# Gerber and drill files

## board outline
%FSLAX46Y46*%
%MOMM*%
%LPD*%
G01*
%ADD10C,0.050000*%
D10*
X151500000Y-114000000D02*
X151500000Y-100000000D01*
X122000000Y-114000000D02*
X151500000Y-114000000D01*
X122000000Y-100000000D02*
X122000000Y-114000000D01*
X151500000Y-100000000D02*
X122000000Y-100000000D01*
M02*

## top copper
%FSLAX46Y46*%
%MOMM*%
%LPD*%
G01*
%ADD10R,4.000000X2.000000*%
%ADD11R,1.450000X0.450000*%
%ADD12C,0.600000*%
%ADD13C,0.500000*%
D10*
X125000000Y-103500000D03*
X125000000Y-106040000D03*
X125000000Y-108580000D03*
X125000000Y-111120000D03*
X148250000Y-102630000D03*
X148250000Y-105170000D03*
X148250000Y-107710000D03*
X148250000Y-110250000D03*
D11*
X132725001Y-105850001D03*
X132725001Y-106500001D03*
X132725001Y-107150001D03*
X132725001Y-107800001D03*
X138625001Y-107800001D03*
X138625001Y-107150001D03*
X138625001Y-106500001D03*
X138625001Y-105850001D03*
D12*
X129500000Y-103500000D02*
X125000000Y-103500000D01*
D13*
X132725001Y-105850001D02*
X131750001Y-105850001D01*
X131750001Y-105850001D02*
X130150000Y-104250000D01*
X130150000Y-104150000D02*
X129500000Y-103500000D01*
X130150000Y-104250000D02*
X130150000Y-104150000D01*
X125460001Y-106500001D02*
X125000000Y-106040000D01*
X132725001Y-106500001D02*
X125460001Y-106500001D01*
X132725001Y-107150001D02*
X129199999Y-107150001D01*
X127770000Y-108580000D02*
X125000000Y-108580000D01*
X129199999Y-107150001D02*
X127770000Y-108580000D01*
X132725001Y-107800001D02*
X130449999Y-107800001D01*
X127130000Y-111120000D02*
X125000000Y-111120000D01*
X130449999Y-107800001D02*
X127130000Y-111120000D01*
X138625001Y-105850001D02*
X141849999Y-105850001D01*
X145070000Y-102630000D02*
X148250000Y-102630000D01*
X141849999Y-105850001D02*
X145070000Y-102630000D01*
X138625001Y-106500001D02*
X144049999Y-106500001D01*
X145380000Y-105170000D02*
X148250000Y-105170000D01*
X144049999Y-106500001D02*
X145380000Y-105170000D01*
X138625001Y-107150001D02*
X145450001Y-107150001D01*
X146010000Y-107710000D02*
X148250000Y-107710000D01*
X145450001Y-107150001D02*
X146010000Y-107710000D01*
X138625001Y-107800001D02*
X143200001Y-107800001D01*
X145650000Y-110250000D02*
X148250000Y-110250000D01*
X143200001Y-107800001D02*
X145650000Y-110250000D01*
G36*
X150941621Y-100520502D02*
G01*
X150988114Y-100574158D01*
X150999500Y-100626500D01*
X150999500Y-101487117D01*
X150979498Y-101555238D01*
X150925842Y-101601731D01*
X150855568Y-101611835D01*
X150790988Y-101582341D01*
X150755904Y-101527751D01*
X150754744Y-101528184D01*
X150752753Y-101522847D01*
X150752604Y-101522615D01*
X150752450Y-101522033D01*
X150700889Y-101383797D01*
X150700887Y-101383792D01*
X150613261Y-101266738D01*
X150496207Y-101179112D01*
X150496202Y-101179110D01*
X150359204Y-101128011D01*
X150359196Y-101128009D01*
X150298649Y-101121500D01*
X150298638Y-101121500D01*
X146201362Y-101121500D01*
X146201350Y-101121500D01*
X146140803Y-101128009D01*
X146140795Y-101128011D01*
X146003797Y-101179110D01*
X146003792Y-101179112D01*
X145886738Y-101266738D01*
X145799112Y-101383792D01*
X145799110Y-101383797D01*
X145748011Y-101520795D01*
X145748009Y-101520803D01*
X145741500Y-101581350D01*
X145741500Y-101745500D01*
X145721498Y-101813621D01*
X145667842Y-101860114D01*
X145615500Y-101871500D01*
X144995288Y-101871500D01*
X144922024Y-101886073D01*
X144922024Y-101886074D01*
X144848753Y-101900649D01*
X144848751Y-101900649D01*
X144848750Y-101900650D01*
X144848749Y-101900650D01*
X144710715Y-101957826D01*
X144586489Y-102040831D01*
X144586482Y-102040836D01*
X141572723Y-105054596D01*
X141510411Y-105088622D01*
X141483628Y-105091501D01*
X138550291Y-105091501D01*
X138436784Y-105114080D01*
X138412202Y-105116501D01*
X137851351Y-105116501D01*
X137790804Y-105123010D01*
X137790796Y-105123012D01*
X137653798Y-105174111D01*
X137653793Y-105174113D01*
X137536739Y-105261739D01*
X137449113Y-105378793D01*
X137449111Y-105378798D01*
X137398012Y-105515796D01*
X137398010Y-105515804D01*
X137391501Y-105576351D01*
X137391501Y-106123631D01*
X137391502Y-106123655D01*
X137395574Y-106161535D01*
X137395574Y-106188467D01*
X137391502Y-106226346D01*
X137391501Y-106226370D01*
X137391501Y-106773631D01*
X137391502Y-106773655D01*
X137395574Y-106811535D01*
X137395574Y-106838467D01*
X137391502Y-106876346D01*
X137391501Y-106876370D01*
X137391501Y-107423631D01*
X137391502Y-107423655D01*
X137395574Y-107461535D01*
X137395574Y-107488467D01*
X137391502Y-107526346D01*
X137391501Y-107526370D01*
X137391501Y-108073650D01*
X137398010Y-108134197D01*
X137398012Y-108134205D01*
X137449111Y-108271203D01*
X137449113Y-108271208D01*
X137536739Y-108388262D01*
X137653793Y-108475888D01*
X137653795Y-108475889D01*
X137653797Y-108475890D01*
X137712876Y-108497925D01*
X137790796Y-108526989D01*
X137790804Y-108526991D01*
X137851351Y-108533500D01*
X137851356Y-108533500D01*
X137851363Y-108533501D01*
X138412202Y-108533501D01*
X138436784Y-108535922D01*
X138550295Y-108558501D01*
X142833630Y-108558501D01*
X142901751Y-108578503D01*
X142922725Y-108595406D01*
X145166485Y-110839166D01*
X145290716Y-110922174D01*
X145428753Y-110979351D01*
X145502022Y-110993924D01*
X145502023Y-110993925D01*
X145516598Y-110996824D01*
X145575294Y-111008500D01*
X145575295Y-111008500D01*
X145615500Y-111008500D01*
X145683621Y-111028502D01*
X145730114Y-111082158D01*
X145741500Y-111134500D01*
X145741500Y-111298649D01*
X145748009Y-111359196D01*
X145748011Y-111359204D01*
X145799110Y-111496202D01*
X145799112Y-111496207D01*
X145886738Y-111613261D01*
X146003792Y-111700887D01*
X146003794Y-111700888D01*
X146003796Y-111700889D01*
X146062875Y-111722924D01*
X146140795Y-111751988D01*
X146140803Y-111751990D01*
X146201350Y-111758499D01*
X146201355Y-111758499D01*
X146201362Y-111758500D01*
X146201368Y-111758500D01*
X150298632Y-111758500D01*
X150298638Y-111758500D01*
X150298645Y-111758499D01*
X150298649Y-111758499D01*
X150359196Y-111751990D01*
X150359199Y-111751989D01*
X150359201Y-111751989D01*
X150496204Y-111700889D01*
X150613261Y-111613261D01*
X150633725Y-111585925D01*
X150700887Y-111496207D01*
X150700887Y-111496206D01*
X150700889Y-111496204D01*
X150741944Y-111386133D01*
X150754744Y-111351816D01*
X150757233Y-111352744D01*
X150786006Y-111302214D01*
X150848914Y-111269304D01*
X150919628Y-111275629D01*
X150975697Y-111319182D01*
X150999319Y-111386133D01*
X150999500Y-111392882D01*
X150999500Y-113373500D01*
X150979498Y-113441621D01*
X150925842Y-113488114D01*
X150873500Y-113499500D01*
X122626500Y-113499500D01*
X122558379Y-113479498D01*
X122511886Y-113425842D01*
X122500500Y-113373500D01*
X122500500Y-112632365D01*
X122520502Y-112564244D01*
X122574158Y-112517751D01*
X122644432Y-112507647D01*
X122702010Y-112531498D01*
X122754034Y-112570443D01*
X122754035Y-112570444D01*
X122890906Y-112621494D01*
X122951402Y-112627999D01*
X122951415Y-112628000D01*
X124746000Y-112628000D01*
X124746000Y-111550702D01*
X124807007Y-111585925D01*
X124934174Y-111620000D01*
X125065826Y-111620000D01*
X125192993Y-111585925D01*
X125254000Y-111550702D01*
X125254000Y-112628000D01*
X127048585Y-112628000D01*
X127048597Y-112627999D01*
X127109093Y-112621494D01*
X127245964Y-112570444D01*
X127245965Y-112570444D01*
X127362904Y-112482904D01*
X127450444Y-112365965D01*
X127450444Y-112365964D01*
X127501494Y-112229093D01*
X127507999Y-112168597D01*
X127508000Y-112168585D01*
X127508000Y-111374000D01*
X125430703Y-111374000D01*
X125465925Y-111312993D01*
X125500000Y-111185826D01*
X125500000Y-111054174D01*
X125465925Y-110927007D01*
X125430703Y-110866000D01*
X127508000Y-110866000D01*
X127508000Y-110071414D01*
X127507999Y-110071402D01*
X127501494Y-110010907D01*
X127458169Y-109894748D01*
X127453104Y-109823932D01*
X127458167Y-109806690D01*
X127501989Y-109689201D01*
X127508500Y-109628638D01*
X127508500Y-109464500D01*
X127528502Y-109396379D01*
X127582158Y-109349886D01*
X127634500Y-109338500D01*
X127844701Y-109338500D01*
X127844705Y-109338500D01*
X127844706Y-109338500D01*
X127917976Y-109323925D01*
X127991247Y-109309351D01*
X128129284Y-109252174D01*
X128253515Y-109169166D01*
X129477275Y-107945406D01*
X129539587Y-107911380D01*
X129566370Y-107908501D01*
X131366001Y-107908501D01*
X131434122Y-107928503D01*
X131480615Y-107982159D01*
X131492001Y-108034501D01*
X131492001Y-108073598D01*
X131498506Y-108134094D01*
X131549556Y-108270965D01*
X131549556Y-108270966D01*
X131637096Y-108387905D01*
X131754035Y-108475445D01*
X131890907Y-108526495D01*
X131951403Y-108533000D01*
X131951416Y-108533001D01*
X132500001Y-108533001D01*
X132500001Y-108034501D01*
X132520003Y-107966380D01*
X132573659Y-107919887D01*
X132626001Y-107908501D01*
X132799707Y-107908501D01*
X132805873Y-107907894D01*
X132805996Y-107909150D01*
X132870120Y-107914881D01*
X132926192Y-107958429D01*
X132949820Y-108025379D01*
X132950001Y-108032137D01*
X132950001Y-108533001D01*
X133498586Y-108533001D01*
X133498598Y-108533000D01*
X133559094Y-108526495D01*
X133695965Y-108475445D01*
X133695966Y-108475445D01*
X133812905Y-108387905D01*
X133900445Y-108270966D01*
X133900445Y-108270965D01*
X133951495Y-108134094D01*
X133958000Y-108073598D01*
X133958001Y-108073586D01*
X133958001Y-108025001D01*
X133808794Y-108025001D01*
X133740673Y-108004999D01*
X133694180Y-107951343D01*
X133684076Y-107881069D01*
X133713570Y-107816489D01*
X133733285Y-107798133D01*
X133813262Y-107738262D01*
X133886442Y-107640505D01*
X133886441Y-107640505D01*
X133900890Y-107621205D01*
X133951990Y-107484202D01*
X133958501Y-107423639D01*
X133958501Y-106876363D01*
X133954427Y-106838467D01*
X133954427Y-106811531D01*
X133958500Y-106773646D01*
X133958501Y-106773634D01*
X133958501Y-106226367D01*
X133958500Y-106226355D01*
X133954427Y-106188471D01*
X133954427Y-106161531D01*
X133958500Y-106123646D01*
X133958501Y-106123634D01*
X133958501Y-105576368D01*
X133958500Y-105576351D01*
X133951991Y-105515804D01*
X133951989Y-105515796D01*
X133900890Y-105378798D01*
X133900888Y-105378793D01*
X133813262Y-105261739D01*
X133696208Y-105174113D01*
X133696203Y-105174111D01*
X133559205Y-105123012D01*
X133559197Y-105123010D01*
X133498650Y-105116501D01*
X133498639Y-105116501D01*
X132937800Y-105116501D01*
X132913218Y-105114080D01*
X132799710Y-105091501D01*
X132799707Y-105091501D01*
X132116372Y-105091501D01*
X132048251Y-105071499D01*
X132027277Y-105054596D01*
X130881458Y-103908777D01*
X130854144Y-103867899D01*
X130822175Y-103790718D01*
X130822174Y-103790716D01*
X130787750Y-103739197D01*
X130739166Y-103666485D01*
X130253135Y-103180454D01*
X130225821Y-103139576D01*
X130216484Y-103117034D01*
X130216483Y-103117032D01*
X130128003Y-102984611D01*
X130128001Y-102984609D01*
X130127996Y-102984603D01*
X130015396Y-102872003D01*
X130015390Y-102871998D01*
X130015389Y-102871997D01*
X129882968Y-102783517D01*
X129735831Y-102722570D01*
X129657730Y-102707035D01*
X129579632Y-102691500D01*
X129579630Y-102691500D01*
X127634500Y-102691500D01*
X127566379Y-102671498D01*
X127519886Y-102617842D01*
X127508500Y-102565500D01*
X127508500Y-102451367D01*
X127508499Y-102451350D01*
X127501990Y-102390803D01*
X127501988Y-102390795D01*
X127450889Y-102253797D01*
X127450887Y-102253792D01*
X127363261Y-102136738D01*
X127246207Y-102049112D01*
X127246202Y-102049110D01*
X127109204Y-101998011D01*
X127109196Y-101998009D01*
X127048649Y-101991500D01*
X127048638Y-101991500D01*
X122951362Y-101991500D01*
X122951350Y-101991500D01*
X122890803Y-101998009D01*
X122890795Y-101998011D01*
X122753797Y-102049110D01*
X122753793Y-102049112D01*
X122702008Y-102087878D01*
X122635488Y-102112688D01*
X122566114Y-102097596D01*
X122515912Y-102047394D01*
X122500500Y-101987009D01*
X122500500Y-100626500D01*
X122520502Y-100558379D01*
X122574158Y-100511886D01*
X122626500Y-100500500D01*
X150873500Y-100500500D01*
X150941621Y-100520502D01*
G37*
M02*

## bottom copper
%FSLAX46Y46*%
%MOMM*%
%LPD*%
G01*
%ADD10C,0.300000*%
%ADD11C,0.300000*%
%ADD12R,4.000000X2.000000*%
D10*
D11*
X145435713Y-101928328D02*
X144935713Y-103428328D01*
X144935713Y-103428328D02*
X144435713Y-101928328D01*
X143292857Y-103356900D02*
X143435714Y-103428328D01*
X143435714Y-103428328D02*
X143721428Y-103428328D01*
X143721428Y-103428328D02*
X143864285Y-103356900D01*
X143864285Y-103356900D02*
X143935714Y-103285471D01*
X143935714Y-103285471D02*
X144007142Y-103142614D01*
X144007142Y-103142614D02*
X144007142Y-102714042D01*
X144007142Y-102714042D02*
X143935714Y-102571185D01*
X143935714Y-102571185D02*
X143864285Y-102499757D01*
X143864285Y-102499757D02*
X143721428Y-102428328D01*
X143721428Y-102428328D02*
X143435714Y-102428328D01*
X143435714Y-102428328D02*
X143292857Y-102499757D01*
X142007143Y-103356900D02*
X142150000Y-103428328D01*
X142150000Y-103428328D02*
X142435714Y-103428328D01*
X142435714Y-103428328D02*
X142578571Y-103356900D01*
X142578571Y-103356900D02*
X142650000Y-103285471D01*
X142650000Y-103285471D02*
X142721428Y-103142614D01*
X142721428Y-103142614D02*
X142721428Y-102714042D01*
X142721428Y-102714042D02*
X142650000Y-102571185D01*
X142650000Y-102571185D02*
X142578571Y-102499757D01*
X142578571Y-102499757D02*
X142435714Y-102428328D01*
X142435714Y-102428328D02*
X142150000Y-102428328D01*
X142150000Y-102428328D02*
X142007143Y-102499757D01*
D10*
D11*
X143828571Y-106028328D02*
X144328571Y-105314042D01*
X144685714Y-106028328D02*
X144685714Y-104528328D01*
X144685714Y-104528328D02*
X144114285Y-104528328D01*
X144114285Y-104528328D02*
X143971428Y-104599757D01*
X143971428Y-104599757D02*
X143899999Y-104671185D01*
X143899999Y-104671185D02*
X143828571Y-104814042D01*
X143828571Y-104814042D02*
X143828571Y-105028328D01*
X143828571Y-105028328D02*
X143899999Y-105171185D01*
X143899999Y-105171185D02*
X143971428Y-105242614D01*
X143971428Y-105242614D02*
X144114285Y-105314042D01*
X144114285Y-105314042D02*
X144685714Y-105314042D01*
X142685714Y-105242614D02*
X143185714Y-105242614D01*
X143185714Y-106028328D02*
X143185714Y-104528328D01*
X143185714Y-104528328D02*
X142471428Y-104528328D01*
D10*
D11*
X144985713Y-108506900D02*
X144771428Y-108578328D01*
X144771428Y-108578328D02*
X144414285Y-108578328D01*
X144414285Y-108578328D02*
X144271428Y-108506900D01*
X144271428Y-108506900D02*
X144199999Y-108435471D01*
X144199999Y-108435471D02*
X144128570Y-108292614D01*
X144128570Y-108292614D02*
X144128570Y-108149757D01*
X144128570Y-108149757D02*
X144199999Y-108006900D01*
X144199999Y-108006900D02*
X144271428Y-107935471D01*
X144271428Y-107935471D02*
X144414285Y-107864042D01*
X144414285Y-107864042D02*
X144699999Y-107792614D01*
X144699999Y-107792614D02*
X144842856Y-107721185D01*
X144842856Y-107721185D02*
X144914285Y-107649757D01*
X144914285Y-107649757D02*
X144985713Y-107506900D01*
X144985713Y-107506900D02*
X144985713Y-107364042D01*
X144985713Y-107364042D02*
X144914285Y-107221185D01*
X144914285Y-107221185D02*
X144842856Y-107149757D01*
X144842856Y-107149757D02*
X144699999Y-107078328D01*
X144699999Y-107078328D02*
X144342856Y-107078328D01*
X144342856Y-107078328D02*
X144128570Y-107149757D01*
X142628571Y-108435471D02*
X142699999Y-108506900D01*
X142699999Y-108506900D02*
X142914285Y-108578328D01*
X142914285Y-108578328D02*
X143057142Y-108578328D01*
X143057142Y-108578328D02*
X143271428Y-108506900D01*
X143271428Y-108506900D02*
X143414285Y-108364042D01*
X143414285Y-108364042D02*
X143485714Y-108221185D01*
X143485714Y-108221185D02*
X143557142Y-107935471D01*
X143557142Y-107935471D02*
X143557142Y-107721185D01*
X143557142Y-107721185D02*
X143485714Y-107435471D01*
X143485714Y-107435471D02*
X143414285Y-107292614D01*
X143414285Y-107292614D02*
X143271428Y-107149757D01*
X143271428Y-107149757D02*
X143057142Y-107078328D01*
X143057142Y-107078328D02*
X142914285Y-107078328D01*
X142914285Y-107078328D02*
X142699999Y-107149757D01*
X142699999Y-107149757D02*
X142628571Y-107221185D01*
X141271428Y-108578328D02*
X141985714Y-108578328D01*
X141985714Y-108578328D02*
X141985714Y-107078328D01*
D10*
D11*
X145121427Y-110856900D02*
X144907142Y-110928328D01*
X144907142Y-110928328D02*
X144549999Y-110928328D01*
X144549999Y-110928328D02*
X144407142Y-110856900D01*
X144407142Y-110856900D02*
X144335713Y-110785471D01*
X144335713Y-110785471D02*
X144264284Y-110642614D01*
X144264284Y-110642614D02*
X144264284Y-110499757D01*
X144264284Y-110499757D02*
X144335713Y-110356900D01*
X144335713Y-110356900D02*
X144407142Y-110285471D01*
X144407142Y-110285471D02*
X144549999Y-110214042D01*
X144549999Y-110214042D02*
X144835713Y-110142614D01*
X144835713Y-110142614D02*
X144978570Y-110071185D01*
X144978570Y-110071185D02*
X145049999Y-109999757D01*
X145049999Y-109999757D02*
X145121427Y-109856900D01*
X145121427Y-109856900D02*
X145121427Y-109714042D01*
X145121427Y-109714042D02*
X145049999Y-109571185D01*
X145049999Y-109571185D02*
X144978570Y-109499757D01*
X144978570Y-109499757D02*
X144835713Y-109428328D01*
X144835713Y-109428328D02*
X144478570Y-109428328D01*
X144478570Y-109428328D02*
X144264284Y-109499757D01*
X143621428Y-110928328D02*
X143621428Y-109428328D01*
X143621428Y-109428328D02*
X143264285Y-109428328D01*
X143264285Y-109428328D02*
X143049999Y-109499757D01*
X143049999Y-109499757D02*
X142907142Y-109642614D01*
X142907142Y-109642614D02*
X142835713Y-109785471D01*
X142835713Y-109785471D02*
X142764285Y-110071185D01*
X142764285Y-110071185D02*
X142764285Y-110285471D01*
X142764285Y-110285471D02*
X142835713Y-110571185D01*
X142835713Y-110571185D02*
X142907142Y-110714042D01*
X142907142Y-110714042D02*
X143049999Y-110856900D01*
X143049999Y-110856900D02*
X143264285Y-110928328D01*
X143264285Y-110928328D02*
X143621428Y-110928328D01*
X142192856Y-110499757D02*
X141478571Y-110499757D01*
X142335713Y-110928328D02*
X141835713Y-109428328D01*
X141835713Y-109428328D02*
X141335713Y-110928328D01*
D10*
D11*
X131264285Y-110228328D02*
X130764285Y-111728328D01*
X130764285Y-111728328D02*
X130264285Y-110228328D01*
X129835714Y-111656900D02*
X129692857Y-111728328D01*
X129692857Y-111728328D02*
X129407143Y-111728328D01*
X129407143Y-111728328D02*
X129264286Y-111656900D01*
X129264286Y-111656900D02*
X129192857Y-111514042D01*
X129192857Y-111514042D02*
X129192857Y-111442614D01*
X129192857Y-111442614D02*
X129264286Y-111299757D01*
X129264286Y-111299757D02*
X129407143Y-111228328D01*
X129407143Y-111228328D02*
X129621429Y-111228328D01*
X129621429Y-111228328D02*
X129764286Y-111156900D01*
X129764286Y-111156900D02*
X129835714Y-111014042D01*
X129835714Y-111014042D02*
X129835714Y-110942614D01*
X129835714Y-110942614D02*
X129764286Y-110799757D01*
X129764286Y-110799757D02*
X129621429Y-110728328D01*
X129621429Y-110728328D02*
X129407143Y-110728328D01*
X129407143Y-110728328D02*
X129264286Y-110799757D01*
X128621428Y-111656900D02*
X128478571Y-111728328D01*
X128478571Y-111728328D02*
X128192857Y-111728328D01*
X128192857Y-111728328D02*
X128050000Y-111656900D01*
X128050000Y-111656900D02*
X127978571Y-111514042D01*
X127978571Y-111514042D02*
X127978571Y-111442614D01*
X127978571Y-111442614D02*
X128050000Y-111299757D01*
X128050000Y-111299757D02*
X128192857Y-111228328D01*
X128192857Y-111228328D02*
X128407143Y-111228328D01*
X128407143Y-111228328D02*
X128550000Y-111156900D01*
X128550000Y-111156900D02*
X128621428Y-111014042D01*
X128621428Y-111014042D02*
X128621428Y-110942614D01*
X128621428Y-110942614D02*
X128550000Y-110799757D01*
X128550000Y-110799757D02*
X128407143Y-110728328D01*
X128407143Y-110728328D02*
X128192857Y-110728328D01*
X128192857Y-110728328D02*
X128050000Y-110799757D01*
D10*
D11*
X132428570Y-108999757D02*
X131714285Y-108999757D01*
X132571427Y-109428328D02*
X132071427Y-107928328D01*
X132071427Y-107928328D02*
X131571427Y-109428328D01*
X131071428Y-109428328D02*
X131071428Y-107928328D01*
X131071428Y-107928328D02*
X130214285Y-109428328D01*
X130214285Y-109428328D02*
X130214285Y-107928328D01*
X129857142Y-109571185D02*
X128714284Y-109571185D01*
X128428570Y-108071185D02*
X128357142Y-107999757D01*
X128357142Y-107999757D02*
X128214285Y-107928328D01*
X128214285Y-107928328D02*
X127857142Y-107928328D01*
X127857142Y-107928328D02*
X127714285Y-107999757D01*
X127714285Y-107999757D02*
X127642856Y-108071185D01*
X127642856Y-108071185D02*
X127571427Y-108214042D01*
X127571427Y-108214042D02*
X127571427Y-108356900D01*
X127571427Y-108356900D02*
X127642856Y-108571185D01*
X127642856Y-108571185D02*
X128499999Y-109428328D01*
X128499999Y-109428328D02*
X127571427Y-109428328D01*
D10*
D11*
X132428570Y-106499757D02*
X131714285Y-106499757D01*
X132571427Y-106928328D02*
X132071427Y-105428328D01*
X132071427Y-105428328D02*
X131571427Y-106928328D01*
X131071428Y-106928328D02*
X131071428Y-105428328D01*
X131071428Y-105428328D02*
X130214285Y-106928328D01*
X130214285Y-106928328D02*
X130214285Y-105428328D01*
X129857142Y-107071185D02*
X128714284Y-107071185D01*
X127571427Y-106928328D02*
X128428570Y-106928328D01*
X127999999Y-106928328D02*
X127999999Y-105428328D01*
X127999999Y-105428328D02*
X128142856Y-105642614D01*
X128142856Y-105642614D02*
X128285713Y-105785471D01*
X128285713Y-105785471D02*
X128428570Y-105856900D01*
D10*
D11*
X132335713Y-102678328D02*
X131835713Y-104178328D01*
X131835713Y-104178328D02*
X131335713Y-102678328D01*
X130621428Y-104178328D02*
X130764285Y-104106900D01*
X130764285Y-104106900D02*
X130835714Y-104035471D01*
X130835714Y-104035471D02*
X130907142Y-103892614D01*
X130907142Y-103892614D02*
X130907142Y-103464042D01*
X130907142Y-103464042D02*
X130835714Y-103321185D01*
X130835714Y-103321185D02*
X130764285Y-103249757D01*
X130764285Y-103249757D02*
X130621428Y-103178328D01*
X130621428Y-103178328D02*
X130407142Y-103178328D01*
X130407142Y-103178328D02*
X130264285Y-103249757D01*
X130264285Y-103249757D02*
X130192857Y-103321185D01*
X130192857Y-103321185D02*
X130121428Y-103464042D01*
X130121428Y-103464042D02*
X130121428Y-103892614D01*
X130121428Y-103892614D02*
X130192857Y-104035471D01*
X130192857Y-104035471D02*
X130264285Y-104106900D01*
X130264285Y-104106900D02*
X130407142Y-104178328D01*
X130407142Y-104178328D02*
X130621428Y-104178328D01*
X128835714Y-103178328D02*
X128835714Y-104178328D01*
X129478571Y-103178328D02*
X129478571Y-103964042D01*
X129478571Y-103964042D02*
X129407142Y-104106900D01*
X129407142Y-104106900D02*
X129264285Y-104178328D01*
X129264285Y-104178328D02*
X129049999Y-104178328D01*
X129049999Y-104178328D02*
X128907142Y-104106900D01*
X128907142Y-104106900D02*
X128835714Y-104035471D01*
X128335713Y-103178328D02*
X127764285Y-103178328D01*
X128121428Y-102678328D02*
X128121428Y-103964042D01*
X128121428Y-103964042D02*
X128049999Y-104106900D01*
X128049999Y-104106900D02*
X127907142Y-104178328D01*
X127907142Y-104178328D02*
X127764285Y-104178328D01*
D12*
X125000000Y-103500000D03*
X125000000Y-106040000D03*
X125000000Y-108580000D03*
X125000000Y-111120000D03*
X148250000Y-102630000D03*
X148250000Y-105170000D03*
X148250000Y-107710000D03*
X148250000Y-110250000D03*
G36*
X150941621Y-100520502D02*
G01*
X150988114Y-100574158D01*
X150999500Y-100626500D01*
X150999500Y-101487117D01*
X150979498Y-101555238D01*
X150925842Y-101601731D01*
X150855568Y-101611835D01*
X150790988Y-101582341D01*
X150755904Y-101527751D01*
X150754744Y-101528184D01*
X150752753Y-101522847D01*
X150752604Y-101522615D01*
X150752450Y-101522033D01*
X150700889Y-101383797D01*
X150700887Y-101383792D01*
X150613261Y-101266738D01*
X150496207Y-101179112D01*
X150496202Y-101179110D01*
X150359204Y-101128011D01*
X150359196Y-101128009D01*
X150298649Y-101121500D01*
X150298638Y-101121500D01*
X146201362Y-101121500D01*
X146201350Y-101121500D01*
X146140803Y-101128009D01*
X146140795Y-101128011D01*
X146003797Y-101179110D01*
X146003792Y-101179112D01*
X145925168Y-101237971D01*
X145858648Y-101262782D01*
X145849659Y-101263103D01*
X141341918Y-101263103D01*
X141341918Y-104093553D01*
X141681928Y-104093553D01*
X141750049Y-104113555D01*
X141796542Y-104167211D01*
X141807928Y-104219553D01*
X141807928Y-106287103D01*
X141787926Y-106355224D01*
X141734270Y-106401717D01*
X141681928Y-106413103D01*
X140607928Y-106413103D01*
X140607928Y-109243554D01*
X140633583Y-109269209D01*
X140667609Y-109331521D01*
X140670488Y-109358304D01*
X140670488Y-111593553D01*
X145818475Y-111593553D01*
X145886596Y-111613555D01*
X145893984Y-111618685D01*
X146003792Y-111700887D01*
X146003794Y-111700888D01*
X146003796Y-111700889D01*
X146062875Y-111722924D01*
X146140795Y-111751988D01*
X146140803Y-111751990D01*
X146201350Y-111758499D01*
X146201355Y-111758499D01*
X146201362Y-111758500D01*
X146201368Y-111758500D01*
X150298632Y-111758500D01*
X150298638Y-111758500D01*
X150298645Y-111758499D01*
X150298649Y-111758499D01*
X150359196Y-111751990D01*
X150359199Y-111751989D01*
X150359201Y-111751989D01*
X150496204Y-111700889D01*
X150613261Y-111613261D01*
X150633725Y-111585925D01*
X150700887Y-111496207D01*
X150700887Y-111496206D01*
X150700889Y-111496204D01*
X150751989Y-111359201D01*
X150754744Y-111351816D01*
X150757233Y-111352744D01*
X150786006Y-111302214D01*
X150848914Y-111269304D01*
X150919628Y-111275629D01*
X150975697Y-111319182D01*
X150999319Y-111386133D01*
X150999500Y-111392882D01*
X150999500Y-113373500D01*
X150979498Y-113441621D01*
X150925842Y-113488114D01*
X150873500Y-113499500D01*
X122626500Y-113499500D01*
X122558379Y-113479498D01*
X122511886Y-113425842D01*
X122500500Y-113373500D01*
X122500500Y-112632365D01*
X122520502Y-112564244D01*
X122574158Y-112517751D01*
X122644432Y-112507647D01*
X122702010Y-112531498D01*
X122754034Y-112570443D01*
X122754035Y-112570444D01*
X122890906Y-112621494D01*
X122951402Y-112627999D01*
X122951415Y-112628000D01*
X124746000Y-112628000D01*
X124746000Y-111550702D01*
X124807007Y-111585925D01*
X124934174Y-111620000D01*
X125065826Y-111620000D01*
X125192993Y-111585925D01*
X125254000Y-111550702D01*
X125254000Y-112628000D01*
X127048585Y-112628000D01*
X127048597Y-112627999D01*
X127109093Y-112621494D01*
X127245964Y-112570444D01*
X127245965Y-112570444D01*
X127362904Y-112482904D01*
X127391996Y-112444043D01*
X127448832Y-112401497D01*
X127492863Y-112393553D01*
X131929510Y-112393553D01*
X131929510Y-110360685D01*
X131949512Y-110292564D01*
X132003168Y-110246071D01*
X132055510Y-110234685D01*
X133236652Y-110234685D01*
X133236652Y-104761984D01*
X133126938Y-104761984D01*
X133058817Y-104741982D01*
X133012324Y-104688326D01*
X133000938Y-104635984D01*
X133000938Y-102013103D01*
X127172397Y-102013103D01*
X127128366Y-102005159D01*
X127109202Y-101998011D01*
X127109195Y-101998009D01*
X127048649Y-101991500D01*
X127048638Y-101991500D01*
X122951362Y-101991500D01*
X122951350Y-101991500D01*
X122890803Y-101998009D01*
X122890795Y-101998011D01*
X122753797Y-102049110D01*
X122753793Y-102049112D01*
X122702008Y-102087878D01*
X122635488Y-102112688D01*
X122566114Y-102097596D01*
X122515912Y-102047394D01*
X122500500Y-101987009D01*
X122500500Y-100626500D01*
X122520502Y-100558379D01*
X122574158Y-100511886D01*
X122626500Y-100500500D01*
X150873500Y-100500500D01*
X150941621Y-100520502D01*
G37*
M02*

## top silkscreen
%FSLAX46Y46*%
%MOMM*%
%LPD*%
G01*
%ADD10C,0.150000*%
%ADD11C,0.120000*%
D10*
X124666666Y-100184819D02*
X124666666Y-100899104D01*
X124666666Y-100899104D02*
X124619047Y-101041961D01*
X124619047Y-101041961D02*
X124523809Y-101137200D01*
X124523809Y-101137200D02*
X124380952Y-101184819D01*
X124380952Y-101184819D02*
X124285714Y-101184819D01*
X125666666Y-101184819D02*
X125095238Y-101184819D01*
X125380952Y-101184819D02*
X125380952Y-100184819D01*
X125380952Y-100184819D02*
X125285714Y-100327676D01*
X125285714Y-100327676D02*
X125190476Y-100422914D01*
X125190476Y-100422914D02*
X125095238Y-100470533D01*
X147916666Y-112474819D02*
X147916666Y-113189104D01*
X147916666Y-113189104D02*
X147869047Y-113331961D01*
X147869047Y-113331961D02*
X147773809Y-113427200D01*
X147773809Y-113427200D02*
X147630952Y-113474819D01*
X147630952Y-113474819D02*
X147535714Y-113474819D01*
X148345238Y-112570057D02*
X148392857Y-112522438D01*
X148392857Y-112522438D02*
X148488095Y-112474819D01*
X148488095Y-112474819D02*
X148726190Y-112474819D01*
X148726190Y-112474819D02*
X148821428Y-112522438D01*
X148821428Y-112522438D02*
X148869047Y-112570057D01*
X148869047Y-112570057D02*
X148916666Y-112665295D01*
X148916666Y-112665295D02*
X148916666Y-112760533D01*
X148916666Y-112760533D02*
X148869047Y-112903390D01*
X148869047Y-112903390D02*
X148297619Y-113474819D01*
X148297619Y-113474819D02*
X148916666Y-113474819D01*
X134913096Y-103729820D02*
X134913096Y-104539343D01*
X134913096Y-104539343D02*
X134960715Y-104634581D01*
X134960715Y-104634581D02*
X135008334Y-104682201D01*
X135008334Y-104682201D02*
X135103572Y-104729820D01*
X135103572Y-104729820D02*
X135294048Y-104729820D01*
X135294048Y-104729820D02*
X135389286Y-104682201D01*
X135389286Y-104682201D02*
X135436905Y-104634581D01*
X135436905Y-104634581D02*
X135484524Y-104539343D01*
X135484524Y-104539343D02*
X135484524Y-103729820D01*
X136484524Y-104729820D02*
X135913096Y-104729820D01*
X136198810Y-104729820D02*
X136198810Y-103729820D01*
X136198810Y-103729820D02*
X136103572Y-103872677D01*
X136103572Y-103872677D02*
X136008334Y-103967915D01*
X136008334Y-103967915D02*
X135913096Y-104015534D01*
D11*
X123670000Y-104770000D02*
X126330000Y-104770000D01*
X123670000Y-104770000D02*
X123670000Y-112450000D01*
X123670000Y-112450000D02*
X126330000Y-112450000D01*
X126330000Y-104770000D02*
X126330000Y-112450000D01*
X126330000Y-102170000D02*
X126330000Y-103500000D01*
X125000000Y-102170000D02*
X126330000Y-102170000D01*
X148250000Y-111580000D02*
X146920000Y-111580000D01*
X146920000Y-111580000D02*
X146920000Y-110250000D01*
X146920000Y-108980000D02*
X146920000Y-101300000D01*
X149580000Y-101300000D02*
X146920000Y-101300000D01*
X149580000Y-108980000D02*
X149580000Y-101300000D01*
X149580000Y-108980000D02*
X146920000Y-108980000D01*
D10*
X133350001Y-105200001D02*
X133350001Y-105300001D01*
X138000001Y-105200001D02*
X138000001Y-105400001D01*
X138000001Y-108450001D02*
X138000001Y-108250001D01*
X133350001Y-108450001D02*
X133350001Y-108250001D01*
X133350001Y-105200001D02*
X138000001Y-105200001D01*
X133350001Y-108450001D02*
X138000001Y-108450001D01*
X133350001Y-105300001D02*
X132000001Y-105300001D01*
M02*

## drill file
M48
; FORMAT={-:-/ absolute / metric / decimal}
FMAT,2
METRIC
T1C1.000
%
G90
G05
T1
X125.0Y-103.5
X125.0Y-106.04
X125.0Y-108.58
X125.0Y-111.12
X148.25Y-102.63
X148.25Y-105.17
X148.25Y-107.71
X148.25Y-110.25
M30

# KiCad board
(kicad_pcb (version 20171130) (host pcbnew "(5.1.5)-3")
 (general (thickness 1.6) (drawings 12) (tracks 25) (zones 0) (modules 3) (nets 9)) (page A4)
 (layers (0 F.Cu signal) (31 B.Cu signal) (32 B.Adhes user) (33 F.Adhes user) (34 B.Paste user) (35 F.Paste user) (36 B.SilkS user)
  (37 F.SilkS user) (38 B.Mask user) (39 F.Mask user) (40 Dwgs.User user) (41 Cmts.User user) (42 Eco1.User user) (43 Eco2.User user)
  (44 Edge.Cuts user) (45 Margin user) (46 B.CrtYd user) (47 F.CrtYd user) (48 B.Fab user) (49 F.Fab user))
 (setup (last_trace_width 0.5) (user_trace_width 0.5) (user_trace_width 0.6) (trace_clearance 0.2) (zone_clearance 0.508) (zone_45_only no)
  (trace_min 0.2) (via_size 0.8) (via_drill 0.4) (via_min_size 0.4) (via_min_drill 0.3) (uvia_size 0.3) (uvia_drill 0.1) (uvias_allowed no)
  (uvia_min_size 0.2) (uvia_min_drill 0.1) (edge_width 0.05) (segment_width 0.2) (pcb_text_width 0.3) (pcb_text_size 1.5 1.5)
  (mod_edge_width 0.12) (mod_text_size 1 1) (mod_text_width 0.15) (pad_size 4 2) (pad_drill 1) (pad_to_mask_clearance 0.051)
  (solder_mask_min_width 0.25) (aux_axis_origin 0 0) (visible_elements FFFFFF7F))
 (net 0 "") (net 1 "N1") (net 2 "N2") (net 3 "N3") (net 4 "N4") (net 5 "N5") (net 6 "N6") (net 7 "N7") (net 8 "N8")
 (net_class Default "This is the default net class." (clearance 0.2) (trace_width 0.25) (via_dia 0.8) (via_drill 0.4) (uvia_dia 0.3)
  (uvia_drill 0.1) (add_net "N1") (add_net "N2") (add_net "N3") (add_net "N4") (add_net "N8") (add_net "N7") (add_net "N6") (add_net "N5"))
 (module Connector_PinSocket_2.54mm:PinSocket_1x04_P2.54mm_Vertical (layer F.Cu) (at 125 103.5)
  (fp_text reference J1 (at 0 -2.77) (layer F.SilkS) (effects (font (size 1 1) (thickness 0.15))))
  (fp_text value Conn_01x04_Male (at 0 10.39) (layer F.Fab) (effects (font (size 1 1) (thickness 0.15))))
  (fp_line (start -1.33 1.27) (end 1.33 1.27) (layer F.SilkS) (width 0.12))
  (fp_line (start -1.33 1.27) (end -1.33 8.95) (layer F.SilkS) (width 0.12))
  (fp_line (start -1.33 8.95) (end 1.33 8.95) (layer F.SilkS) (width 0.12))
  (fp_line (start 1.33 1.27) (end 1.33 8.95) (layer F.SilkS) (width 0.12))
  (fp_line (start 1.33 -1.33) (end 1.33 0) (layer F.SilkS) (width 0.12))
  (fp_line (start 0 -1.33) (end 1.33 -1.33) (layer F.SilkS) (width 0.12))
  (pad 1 thru_hole rect (at 0 0) (size 4 2) (drill 1) (layers *.Cu *.Mask) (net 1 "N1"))
  (pad 2 thru_hole rect (at 0 2.54) (size 4 2) (drill 1) (layers *.Cu *.Mask) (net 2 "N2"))
  (pad 3 thru_hole rect (at 0 5.08) (size 4 2) (drill 1) (layers *.Cu *.Mask) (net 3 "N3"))
  (pad 4 thru_hole rect (at 0 7.62) (size 4 2) (drill 1) (layers *.Cu *.Mask) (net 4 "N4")))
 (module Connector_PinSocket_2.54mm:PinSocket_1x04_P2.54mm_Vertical (layer F.Cu) (at 148.25 110.25 180)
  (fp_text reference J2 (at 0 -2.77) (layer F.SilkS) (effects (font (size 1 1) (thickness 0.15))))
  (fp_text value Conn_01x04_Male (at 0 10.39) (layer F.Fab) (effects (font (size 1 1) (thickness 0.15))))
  (fp_line (start 0 -1.33) (end 1.33 -1.33) (layer F.SilkS) (width 0.12))
  (fp_line (start 1.33 -1.33) (end 1.33 0) (layer F.SilkS) (width 0.12))
  (fp_line (start 1.33 1.27) (end 1.33 8.95) (layer F.SilkS) (width 0.12))
  (fp_line (start -1.33 8.95) (end 1.33 8.95) (layer F.SilkS) (width 0.12))
  (fp_line (start -1.33 1.27) (end -1.33 8.95) (layer F.SilkS) (width 0.12))
  (fp_line (start -1.33 1.27) (end 1.33 1.27) (layer F.SilkS) (width 0.12))
  (pad 4 thru_hole rect (at 0 7.62 180) (size 4 2) (drill 1) (layers *.Cu *.Mask) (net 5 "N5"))
  (pad 3 thru_hole rect (at 0 5.08 180) (size 4 2) (drill 1) (layers *.Cu *.Mask) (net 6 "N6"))
  (pad 2 thru_hole rect (at 0 2.54 180) (size 4 2) (drill 1) (layers *.Cu *.Mask) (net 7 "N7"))
  (pad 1 thru_hole rect (at 0 0 180) (size 4 2) (drill 1) (layers *.Cu *.Mask) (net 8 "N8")))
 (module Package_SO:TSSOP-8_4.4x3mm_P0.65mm (layer F.Cu) (at 135.675001 106.825001)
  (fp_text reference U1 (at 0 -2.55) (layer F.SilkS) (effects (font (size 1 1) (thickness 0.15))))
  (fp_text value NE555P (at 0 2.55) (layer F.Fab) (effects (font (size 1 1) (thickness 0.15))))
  (fp_line (start -2.325 -1.625) (end -2.325 -1.525) (layer F.SilkS) (width 0.15))
  (fp_line (start 2.325 -1.625) (end 2.325 -1.425) (layer F.SilkS) (width 0.15))
  (fp_line (start 2.325 1.625) (end 2.325 1.425) (layer F.SilkS) (width 0.15))
  (fp_line (start -2.325 1.625) (end -2.325 1.425) (layer F.SilkS) (width 0.15))
  (fp_line (start -2.325 -1.625) (end 2.325 -1.625) (layer F.SilkS) (width 0.15))
  (fp_line (start -2.325 1.625) (end 2.325 1.625) (layer F.SilkS) (width 0.15))
  (fp_line (start -2.325 -1.525) (end -3.675 -1.525) (layer F.SilkS) (width 0.15))
  (pad 1 smd rect (at -2.95 -0.975) (size 1.45 0.45) (layers F.Cu F.Paste F.Mask) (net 1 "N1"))
  (pad 2 smd rect (at -2.95 -0.325) (size 1.45 0.45) (layers F.Cu F.Paste F.Mask) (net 2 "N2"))
  (pad 3 smd rect (at -2.95 0.325) (size 1.45 0.45) (layers F.Cu F.Paste F.Mask) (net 3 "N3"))
  (pad 4 smd rect (at -2.95 0.975) (size 1.45 0.45) (layers F.Cu F.Paste F.Mask) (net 4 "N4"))
  (pad 5 smd rect (at 2.95 0.975) (size 1.45 0.45) (layers F.Cu F.Paste F.Mask) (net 8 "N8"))
  (pad 6 smd rect (at 2.95 0.325) (size 1.45 0.45) (layers F.Cu F.Paste F.Mask) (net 7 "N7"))
  (pad 7 smd rect (at 2.95 -0.325) (size 1.45 0.45) (layers F.Cu F.Paste F.Mask) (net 6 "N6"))
  (pad 8 smd rect (at 2.95 -0.975) (size 1.45 0.45) (layers F.Cu F.Paste F.Mask) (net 5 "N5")))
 (gr_line (start 151.5 114) (end 151.5 100) (layer Edge.Cuts) (width 0.05))
 (gr_line (start 122 114) (end 151.5 114) (layer Edge.Cuts) (width 0.05))
 (gr_line (start 122 100) (end 122 114) (layer Edge.Cuts) (width 0.05))
 (gr_line (start 151.5 100) (end 122 100) (layer Edge.Cuts) (width 0.05))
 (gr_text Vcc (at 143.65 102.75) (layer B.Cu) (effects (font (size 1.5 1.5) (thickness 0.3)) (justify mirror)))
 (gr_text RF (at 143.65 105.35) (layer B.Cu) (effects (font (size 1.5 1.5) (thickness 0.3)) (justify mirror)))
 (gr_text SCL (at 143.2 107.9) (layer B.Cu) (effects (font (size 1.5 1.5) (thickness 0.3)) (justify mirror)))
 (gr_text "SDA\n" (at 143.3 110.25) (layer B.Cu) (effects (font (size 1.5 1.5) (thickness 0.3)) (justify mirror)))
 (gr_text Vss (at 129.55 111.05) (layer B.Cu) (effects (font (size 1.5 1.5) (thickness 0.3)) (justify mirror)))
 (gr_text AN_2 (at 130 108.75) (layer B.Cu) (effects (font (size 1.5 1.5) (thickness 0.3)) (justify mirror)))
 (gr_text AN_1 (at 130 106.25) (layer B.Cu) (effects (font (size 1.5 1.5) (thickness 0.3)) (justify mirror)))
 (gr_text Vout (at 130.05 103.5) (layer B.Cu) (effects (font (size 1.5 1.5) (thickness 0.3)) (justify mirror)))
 (segment (start 129.5 103.5) (end 125 103.5) (width 0.6) (layer F.Cu) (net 1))
 (segment (start 132.725001 105.850001) (end 131.750001 105.850001) (width 0.5) (layer F.Cu) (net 1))
 (segment (start 131.750001 105.850001) (end 130.15 104.25) (width 0.5) (layer F.Cu) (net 1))
 (segment (start 130.15 104.15) (end 129.5 103.5) (width 0.5) (layer F.Cu) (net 1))
 (segment (start 130.15 104.25) (end 130.15 104.15) (width 0.5) (layer F.Cu) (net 1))
 (segment (start 125.460001 106.500001) (end 125 106.04) (width 0.5) (layer F.Cu) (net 2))
 (segment (start 132.725001 106.500001) (end 125.460001 106.500001) (width 0.5) (layer F.Cu) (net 2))
 (segment (start 132.725001 107.150001) (end 129.199999 107.150001) (width 0.5) (layer F.Cu) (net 3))
 (segment (start 127.77 108.58) (end 125 108.58) (width 0.5) (layer F.Cu) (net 3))
 (segment (start 129.199999 107.150001) (end 127.77 108.58) (width 0.5) (layer F.Cu) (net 3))
 (segment (start 132.725001 107.800001) (end 130.449999 107.800001) (width 0.5) (layer F.Cu) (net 4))
 (segment (start 127.13 111.12) (end 125 111.12) (width 0.5) (layer F.Cu) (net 4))
 (segment (start 130.449999 107.800001) (end 127.13 111.12) (width 0.5) (layer F.Cu) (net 4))
 (segment (start 138.625001 105.850001) (end 141.849999 105.850001) (width 0.5) (layer F.Cu) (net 5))
 (segment (start 145.07 102.63) (end 148.25 102.63) (width 0.5) (layer F.Cu) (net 5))
 (segment (start 141.849999 105.850001) (end 145.07 102.63) (width 0.5) (layer F.Cu) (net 5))
 (segment (start 138.625001 106.500001) (end 144.049999 106.500001) (width 0.5) (layer F.Cu) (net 6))
 (segment (start 145.38 105.17) (end 148.25 105.17) (width 0.5) (layer F.Cu) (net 6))
 (segment (start 144.049999 106.500001) (end 145.38 105.17) (width 0.5) (layer F.Cu) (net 6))
 (segment (start 138.625001 107.150001) (end 145.450001 107.150001) (width 0.5) (layer F.Cu) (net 7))
 (segment (start 146.01 107.71) (end 148.25 107.71) (width 0.5) (layer F.Cu) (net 7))
 (segment (start 145.450001 107.150001) (end 146.01 107.71) (width 0.5) (layer F.Cu) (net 7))
 (segment (start 138.625001 107.800001) (end 143.200001 107.800001) (width 0.5) (layer F.Cu) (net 8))
 (segment (start 145.65 110.25) (end 148.25 110.25) (width 0.5) (layer F.Cu) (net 8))
 (segment (start 143.200001 107.800001) (end 145.65 110.25) (width 0.5) (layer F.Cu) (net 8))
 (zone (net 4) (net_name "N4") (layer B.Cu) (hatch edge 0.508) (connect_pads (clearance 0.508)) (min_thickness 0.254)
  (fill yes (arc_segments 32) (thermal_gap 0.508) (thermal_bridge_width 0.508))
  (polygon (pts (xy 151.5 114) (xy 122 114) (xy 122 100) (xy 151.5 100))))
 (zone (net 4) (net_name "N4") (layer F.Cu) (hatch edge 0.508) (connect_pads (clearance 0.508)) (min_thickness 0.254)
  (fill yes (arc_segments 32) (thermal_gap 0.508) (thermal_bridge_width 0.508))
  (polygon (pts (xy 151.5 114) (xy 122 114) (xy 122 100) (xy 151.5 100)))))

